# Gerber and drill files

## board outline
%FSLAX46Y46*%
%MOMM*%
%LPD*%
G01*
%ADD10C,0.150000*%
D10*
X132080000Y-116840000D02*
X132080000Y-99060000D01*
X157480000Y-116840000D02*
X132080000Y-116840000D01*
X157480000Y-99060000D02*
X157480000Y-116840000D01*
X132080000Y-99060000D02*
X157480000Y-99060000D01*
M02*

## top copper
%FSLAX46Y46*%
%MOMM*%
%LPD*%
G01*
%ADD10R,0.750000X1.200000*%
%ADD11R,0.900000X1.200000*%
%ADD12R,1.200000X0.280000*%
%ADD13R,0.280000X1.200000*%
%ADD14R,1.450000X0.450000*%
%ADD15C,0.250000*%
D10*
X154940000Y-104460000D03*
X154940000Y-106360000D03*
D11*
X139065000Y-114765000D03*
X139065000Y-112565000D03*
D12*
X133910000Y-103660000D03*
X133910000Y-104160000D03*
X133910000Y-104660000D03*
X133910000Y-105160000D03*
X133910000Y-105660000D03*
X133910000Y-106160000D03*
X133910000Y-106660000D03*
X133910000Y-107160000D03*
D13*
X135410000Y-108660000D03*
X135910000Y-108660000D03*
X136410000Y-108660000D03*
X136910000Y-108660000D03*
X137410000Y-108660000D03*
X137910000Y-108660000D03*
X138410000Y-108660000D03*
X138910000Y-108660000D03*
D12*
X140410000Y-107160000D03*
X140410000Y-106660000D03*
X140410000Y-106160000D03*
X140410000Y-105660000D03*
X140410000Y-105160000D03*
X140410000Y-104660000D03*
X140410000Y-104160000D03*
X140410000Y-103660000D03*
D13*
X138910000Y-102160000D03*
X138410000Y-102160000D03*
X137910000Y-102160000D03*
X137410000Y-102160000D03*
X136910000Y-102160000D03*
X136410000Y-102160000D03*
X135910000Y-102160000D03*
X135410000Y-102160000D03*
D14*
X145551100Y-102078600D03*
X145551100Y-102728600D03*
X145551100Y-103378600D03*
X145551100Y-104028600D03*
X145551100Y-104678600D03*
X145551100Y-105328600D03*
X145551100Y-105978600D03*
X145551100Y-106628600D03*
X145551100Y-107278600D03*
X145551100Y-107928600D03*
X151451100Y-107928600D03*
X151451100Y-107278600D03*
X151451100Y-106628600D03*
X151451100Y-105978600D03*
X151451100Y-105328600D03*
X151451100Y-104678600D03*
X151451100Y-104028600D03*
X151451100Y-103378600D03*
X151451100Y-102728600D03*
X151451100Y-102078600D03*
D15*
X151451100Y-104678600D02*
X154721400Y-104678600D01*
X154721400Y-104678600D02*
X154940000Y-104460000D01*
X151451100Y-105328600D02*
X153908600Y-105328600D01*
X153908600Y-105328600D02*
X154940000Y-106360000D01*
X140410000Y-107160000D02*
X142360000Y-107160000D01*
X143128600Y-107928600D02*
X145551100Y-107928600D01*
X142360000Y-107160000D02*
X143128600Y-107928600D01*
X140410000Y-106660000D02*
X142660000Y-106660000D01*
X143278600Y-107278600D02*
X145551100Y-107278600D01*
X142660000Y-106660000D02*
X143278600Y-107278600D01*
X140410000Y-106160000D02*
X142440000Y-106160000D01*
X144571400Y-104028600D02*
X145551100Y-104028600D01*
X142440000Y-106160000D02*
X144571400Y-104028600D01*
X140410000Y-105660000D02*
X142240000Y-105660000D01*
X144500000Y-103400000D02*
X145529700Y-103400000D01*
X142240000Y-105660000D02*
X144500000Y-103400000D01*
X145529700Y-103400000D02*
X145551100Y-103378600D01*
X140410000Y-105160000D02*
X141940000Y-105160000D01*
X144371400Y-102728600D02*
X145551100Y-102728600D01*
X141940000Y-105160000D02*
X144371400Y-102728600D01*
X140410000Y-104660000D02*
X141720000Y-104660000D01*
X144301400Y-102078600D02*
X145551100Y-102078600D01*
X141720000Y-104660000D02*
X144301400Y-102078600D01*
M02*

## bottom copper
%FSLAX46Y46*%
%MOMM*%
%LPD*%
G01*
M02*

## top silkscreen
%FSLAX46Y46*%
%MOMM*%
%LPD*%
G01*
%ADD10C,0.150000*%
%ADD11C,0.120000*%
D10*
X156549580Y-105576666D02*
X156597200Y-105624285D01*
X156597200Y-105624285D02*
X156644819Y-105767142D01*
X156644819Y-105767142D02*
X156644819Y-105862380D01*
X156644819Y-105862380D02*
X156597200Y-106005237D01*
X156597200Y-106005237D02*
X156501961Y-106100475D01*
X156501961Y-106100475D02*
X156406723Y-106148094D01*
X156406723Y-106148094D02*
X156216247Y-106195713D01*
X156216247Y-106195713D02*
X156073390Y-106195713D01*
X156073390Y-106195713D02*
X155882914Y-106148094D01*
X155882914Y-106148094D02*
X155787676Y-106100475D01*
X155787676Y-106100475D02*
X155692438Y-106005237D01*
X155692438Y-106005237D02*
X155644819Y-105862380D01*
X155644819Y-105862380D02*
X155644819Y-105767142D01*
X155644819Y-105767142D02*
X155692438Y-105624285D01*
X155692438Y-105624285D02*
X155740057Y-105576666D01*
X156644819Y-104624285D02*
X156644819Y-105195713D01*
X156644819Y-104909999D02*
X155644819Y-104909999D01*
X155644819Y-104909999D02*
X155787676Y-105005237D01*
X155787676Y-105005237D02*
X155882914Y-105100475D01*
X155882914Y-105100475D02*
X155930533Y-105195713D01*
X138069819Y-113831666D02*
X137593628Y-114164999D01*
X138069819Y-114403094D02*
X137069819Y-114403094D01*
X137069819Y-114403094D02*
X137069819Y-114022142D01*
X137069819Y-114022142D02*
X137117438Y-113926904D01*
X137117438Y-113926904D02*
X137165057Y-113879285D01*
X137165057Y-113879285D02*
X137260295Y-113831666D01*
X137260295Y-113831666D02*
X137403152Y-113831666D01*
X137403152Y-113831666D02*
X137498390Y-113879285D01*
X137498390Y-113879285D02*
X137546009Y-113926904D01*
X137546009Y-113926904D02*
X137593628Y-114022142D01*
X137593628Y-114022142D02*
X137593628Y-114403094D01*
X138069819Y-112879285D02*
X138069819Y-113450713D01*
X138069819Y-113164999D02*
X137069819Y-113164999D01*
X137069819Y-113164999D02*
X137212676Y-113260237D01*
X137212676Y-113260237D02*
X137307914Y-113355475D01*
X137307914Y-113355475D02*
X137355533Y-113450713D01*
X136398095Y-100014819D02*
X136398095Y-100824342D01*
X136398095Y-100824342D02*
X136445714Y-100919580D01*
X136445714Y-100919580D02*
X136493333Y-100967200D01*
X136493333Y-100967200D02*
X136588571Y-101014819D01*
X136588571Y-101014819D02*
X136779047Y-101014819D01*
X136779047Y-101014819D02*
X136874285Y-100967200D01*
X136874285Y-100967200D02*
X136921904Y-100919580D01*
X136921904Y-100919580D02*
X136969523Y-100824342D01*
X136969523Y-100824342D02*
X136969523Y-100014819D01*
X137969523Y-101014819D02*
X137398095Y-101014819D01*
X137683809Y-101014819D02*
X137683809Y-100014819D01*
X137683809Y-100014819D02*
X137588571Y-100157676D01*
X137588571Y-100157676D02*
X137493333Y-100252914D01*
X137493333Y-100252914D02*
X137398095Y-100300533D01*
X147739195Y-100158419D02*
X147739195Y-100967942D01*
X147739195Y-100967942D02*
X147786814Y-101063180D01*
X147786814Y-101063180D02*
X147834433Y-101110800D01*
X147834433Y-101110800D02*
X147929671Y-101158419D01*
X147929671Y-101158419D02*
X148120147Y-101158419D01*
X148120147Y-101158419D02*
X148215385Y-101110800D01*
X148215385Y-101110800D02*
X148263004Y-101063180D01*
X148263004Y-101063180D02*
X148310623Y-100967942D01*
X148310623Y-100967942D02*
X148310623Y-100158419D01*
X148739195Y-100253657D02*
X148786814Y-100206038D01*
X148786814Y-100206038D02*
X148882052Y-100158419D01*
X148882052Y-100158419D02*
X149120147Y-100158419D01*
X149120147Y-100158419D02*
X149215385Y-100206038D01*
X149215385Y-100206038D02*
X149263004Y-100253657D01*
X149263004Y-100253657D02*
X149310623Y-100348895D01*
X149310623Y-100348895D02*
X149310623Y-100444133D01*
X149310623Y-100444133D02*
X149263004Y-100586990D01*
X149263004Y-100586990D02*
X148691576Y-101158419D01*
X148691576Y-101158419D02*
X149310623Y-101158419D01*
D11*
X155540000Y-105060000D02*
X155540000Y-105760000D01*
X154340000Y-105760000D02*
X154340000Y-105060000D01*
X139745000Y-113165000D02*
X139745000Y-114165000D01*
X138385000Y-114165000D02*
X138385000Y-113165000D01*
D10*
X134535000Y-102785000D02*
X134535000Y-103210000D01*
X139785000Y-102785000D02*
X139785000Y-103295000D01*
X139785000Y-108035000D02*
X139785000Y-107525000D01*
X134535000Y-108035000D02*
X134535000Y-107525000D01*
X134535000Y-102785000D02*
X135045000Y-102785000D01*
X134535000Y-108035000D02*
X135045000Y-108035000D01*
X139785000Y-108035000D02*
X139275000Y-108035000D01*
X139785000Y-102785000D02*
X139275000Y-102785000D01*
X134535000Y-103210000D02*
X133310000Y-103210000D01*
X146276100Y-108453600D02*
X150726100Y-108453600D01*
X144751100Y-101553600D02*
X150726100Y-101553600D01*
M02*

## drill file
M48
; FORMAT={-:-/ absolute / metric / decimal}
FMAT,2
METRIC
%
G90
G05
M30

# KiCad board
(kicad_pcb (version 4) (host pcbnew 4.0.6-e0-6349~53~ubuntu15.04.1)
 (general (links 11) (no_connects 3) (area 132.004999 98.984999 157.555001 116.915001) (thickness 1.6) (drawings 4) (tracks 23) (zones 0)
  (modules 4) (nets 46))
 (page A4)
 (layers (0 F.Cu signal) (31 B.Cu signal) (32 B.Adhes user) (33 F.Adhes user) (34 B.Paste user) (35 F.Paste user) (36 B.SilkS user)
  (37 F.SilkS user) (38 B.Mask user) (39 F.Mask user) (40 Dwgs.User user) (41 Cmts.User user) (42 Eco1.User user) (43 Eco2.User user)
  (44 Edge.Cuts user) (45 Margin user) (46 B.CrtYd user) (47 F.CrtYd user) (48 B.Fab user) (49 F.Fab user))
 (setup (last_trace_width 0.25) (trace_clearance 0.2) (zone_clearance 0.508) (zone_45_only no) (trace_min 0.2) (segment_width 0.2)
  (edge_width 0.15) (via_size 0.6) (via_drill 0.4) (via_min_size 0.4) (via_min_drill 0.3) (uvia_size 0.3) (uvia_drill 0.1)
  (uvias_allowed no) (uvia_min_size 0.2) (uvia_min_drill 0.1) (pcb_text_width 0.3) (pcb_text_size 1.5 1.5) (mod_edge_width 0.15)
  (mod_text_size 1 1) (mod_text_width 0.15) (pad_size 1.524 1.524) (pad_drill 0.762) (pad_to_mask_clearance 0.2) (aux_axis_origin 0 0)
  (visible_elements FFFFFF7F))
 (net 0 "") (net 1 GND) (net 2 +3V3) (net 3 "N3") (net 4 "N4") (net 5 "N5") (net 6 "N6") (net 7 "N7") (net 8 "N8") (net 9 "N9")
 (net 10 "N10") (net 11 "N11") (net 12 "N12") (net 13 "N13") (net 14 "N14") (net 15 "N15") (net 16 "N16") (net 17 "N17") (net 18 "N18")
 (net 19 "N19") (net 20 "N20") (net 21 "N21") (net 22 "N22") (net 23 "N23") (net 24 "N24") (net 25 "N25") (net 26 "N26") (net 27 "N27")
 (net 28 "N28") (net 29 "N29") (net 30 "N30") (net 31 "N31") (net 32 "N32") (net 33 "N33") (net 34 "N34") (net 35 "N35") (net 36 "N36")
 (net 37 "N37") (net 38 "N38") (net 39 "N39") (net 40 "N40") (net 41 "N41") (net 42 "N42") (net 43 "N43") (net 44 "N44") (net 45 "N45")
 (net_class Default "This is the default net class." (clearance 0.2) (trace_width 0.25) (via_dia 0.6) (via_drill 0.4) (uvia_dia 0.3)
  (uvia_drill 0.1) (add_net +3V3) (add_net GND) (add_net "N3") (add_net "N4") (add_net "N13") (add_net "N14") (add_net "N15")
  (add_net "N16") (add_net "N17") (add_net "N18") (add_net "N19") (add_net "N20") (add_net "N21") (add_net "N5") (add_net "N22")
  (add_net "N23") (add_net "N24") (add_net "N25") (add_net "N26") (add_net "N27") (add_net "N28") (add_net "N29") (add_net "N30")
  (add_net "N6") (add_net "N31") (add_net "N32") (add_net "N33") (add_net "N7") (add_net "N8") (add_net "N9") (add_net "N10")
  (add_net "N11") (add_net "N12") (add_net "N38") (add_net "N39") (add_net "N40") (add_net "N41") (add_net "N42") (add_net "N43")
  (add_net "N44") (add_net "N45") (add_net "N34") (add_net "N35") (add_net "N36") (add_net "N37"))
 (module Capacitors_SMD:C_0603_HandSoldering (layer F.Cu) (at 154.94 105.41 270)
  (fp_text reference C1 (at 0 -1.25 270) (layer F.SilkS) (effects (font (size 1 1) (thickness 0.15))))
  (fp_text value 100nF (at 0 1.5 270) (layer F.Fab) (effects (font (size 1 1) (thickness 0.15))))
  (fp_line (start -0.35 -0.6) (end 0.35 -0.6) (layer F.SilkS) (width 0.12))
  (fp_line (start 0.35 0.6) (end -0.35 0.6) (layer F.SilkS) (width 0.12))
  (pad 1 smd rect (at -0.95 0 270) (size 1.2 0.75) (layers F.Cu F.Paste F.Mask) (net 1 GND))
  (pad 2 smd rect (at 0.95 0 270) (size 1.2 0.75) (layers F.Cu F.Paste F.Mask) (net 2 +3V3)))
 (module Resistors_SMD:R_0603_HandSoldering (layer F.Cu) (at 139.065 113.665 90)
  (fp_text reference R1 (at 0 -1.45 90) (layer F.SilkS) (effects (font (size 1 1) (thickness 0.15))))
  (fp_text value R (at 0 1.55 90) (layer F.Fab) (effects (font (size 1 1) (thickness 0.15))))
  (fp_line (start 0.5 0.68) (end -0.5 0.68) (layer F.SilkS) (width 0.12))
  (fp_line (start -0.5 -0.68) (end 0.5 -0.68) (layer F.SilkS) (width 0.12))
  (pad 1 smd rect (at -1.1 0 90) (size 1.2 0.9) (layers F.Cu F.Paste F.Mask) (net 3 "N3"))
  (pad 2 smd rect (at 1.1 0 90) (size 1.2 0.9) (layers F.Cu F.Paste F.Mask) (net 1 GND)))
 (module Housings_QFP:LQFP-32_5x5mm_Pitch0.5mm (layer F.Cu) (at 137.16 105.41)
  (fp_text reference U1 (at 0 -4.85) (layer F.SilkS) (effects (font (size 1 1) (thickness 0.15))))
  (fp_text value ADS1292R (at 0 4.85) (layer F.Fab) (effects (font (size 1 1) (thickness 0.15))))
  (fp_line (start -2.625 -2.625) (end -2.625 -2.2) (layer F.SilkS) (width 0.15))
  (fp_line (start 2.625 -2.625) (end 2.625 -2.115) (layer F.SilkS) (width 0.15))
  (fp_line (start 2.625 2.625) (end 2.625 2.115) (layer F.SilkS) (width 0.15))
  (fp_line (start -2.625 2.625) (end -2.625 2.115) (layer F.SilkS) (width 0.15))
  (fp_line (start -2.625 -2.625) (end -2.115 -2.625) (layer F.SilkS) (width 0.15))
  (fp_line (start -2.625 2.625) (end -2.115 2.625) (layer F.SilkS) (width 0.15))
  (fp_line (start 2.625 2.625) (end 2.115 2.625) (layer F.SilkS) (width 0.15))
  (fp_line (start 2.625 -2.625) (end 2.115 -2.625) (layer F.SilkS) (width 0.15))
  (fp_line (start -2.625 -2.2) (end -3.85 -2.2) (layer F.SilkS) (width 0.15))
  (pad 1 smd rect (at -3.25 -1.75) (size 1.2 0.28) (layers F.Cu F.Paste F.Mask) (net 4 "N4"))
  (pad 2 smd rect (at -3.25 -1.25) (size 1.2 0.28) (layers F.Cu F.Paste F.Mask) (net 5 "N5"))
  (pad 3 smd rect (at -3.25 -0.75) (size 1.2 0.28) (layers F.Cu F.Paste F.Mask) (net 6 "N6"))
  (pad 4 smd rect (at -3.25 -0.25) (size 1.2 0.28) (layers F.Cu F.Paste F.Mask) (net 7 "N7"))
  (pad 5 smd rect (at -3.25 0.25) (size 1.2 0.28) (layers F.Cu F.Paste F.Mask) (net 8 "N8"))
  (pad 6 smd rect (at -3.25 0.75) (size 1.2 0.28) (layers F.Cu F.Paste F.Mask) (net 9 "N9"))
  (pad 7 smd rect (at -3.25 1.25) (size 1.2 0.28) (layers F.Cu F.Paste F.Mask) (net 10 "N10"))
  (pad 8 smd rect (at -3.25 1.75) (size 1.2 0.28) (layers F.Cu F.Paste F.Mask) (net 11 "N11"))
  (pad 9 smd rect (at -1.75 3.25 90) (size 1.2 0.28) (layers F.Cu F.Paste F.Mask) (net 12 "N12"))
  (pad 10 smd rect (at -1.25 3.25 90) (size 1.2 0.28) (layers F.Cu F.Paste F.Mask) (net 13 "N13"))
  (pad 11 smd rect (at -0.75 3.25 90) (size 1.2 0.28) (layers F.Cu F.Paste F.Mask) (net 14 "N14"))
  (pad 12 smd rect (at -0.25 3.25 90) (size 1.2 0.28) (layers F.Cu F.Paste F.Mask) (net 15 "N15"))
  (pad 13 smd rect (at 0.25 3.25 90) (size 1.2 0.28) (layers F.Cu F.Paste F.Mask) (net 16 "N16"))
  (pad 14 smd rect (at 0.75 3.25 90) (size 1.2 0.28) (layers F.Cu F.Paste F.Mask) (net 3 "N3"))
  (pad 15 smd rect (at 1.25 3.25 90) (size 1.2 0.28) (layers F.Cu F.Paste F.Mask) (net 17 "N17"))
  (pad 16 smd rect (at 1.75 3.25 90) (size 1.2 0.28) (layers F.Cu F.Paste F.Mask) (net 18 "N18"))
  (pad 17 smd rect (at 3.25 1.75) (size 1.2 0.28) (layers F.Cu F.Paste F.Mask) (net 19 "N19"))
  (pad 18 smd rect (at 3.25 1.25) (size 1.2 0.28) (layers F.Cu F.Paste F.Mask) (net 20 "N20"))
  (pad 19 smd rect (at 3.25 0.75) (size 1.2 0.28) (layers F.Cu F.Paste F.Mask) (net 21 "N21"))
  (pad 20 smd rect (at 3.25 0.25) (size 1.2 0.28) (layers F.Cu F.Paste F.Mask) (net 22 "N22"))
  (pad 21 smd rect (at 3.25 -0.25) (size 1.2 0.28) (layers F.Cu F.Paste F.Mask) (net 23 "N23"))
  (pad 22 smd rect (at 3.25 -0.75) (size 1.2 0.28) (layers F.Cu F.Paste F.Mask) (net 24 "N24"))
  (pad 23 smd rect (at 3.25 -1.25) (size 1.2 0.28) (layers F.Cu F.Paste F.Mask) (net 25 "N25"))
  (pad 24 smd rect (at 3.25 -1.75) (size 1.2 0.28) (layers F.Cu F.Paste F.Mask) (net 1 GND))
  (pad 25 smd rect (at 1.75 -3.25 90) (size 1.2 0.28) (layers F.Cu F.Paste F.Mask) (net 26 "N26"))
  (pad 26 smd rect (at 1.25 -3.25 90) (size 1.2 0.28) (layers F.Cu F.Paste F.Mask) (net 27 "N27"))
  (pad 27 smd rect (at 0.75 -3.25 90) (size 1.2 0.28) (layers F.Cu F.Paste F.Mask) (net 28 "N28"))
  (pad 28 smd rect (at 0.25 -3.25 90) (size 1.2 0.28) (layers F.Cu F.Paste F.Mask) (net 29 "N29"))
  (pad 29 smd rect (at -0.25 -3.25 90) (size 1.2 0.28) (layers F.Cu F.Paste F.Mask) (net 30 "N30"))
  (pad 30 smd rect (at -0.75 -3.25 90) (size 1.2 0.28) (layers F.Cu F.Paste F.Mask) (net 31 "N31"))
  (pad 31 smd rect (at -1.25 -3.25 90) (size 1.2 0.28) (layers F.Cu F.Paste F.Mask) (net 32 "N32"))
  (pad 32 smd rect (at -1.75 -3.25 90) (size 1.2 0.28) (layers F.Cu F.Paste F.Mask) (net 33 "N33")))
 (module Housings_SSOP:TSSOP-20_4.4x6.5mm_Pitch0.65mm (layer F.Cu) (at 148.5011 105.0036)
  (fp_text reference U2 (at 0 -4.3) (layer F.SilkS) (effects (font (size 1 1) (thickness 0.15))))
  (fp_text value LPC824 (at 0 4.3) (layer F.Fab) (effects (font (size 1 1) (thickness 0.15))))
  (fp_line (start -2.225 3.45) (end 2.225 3.45) (layer F.SilkS) (width 0.15))
  (fp_line (start -3.75 -3.45) (end 2.225 -3.45) (layer F.SilkS) (width 0.15))
  (pad 1 smd rect (at -2.95 -2.925) (size 1.45 0.45) (layers F.Cu F.Paste F.Mask) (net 24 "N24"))
  (pad 2 smd rect (at -2.95 -2.275) (size 1.45 0.45) (layers F.Cu F.Paste F.Mask) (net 23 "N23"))
  (pad 3 smd rect (at -2.95 -1.625) (size 1.45 0.45) (layers F.Cu F.Paste F.Mask) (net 22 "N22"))
  (pad 4 smd rect (at -2.95 -0.975) (size 1.45 0.45) (layers F.Cu F.Paste F.Mask) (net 21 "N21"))
  (pad 5 smd rect (at -2.95 -0.325) (size 1.45 0.45) (layers F.Cu F.Paste F.Mask) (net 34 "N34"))
  (pad 6 smd rect (at -2.95 0.325) (size 1.45 0.45) (layers F.Cu F.Paste F.Mask) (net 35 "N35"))
  (pad 7 smd rect (at -2.95 0.975) (size 1.45 0.45) (layers F.Cu F.Paste F.Mask) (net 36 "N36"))
  (pad 8 smd rect (at -2.95 1.625) (size 1.45 0.45) (layers F.Cu F.Paste F.Mask) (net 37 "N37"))
  (pad 9 smd rect (at -2.95 2.275) (size 1.45 0.45) (layers F.Cu F.Paste F.Mask) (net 20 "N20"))
  (pad 10 smd rect (at -2.95 2.925) (size 1.45 0.45) (layers F.Cu F.Paste F.Mask) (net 19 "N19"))
  (pad 11 smd rect (at 2.95 2.925) (size 1.45 0.45) (layers F.Cu F.Paste F.Mask) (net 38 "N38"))
  (pad 12 smd rect (at 2.95 2.275) (size 1.45 0.45) (layers F.Cu F.Paste F.Mask) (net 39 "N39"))
  (pad 13 smd rect (at 2.95 1.625) (size 1.45 0.45) (layers F.Cu F.Paste F.Mask) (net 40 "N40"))
  (pad 14 smd rect (at 2.95 0.975) (size 1.45 0.45) (layers F.Cu F.Paste F.Mask) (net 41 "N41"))
  (pad 15 smd rect (at 2.95 0.325) (size 1.45 0.45) (layers F.Cu F.Paste F.Mask) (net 2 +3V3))
  (pad 16 smd rect (at 2.95 -0.325) (size 1.45 0.45) (layers F.Cu F.Paste F.Mask) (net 1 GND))
  (pad 17 smd rect (at 2.95 -0.975) (size 1.45 0.45) (layers F.Cu F.Paste F.Mask) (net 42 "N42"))
  (pad 18 smd rect (at 2.95 -1.625) (size 1.45 0.45) (layers F.Cu F.Paste F.Mask) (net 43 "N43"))
  (pad 19 smd rect (at 2.95 -2.275) (size 1.45 0.45) (layers F.Cu F.Paste F.Mask) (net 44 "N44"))
  (pad 20 smd rect (at 2.95 -2.925) (size 1.45 0.45) (layers F.Cu F.Paste F.Mask) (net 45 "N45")))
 (gr_line (start 132.08 116.84) (end 132.08 99.06) (angle 90) (layer Edge.Cuts) (width 0.15))
 (gr_line (start 157.48 116.84) (end 132.08 116.84) (angle 90) (layer Edge.Cuts) (width 0.15))
 (gr_line (start 157.48 99.06) (end 157.48 116.84) (angle 90) (layer Edge.Cuts) (width 0.15))
 (gr_line (start 132.08 99.06) (end 157.48 99.06) (angle 90) (layer Edge.Cuts) (width 0.15))
 (segment (start 151.4511 104.6786) (end 154.7214 104.6786) (width 0.25) (layer F.Cu) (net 1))
 (segment (start 154.7214 104.6786) (end 154.94 104.46) (width 0.25) (layer F.Cu) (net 1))
 (segment (start 151.4511 105.3286) (end 153.9086 105.3286) (width 0.25) (layer F.Cu) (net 2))
 (segment (start 153.9086 105.3286) (end 154.94 106.36) (width 0.25) (layer F.Cu) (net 2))
 (segment (start 140.41 107.16) (end 142.36 107.16) (width 0.25) (layer F.Cu) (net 19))
 (segment (start 143.1286 107.9286) (end 145.5511 107.9286) (width 0.25) (layer F.Cu) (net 19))
 (segment (start 142.36 107.16) (end 143.1286 107.9286) (width 0.25) (layer F.Cu) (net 19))
 (segment (start 140.41 106.66) (end 142.66 106.66) (width 0.25) (layer F.Cu) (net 20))
 (segment (start 143.2786 107.2786) (end 145.5511 107.2786) (width 0.25) (layer F.Cu) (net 20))
 (segment (start 142.66 106.66) (end 143.2786 107.2786) (width 0.25) (layer F.Cu) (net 20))
 (segment (start 140.41 106.16) (end 142.44 106.16) (width 0.25) (layer F.Cu) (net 21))
 (segment (start 144.5714 104.0286) (end 145.5511 104.0286) (width 0.25) (layer F.Cu) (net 21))
 (segment (start 142.44 106.16) (end 144.5714 104.0286) (width 0.25) (layer F.Cu) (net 21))
 (segment (start 140.41 105.66) (end 142.24 105.66) (width 0.25) (layer F.Cu) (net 22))
 (segment (start 144.5 103.4) (end 145.5297 103.4) (width 0.25) (layer F.Cu) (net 22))
 (segment (start 142.24 105.66) (end 144.5 103.4) (width 0.25) (layer F.Cu) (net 22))
 (segment (start 145.5297 103.4) (end 145.5511 103.3786) (width 0.25) (layer F.Cu) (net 22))
 (segment (start 140.41 105.16) (end 141.94 105.16) (width 0.25) (layer F.Cu) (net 23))
 (segment (start 144.3714 102.7286) (end 145.5511 102.7286) (width 0.25) (layer F.Cu) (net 23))
 (segment (start 141.94 105.16) (end 144.3714 102.7286) (width 0.25) (layer F.Cu) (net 23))
 (segment (start 140.41 104.66) (end 141.72 104.66) (width 0.25) (layer F.Cu) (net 24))
 (segment (start 144.3014 102.0786) (end 145.5511 102.0786) (width 0.25) (layer F.Cu) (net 24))
 (segment (start 141.72 104.66) (end 144.3014 102.0786) (width 0.25) (layer F.Cu) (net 24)))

